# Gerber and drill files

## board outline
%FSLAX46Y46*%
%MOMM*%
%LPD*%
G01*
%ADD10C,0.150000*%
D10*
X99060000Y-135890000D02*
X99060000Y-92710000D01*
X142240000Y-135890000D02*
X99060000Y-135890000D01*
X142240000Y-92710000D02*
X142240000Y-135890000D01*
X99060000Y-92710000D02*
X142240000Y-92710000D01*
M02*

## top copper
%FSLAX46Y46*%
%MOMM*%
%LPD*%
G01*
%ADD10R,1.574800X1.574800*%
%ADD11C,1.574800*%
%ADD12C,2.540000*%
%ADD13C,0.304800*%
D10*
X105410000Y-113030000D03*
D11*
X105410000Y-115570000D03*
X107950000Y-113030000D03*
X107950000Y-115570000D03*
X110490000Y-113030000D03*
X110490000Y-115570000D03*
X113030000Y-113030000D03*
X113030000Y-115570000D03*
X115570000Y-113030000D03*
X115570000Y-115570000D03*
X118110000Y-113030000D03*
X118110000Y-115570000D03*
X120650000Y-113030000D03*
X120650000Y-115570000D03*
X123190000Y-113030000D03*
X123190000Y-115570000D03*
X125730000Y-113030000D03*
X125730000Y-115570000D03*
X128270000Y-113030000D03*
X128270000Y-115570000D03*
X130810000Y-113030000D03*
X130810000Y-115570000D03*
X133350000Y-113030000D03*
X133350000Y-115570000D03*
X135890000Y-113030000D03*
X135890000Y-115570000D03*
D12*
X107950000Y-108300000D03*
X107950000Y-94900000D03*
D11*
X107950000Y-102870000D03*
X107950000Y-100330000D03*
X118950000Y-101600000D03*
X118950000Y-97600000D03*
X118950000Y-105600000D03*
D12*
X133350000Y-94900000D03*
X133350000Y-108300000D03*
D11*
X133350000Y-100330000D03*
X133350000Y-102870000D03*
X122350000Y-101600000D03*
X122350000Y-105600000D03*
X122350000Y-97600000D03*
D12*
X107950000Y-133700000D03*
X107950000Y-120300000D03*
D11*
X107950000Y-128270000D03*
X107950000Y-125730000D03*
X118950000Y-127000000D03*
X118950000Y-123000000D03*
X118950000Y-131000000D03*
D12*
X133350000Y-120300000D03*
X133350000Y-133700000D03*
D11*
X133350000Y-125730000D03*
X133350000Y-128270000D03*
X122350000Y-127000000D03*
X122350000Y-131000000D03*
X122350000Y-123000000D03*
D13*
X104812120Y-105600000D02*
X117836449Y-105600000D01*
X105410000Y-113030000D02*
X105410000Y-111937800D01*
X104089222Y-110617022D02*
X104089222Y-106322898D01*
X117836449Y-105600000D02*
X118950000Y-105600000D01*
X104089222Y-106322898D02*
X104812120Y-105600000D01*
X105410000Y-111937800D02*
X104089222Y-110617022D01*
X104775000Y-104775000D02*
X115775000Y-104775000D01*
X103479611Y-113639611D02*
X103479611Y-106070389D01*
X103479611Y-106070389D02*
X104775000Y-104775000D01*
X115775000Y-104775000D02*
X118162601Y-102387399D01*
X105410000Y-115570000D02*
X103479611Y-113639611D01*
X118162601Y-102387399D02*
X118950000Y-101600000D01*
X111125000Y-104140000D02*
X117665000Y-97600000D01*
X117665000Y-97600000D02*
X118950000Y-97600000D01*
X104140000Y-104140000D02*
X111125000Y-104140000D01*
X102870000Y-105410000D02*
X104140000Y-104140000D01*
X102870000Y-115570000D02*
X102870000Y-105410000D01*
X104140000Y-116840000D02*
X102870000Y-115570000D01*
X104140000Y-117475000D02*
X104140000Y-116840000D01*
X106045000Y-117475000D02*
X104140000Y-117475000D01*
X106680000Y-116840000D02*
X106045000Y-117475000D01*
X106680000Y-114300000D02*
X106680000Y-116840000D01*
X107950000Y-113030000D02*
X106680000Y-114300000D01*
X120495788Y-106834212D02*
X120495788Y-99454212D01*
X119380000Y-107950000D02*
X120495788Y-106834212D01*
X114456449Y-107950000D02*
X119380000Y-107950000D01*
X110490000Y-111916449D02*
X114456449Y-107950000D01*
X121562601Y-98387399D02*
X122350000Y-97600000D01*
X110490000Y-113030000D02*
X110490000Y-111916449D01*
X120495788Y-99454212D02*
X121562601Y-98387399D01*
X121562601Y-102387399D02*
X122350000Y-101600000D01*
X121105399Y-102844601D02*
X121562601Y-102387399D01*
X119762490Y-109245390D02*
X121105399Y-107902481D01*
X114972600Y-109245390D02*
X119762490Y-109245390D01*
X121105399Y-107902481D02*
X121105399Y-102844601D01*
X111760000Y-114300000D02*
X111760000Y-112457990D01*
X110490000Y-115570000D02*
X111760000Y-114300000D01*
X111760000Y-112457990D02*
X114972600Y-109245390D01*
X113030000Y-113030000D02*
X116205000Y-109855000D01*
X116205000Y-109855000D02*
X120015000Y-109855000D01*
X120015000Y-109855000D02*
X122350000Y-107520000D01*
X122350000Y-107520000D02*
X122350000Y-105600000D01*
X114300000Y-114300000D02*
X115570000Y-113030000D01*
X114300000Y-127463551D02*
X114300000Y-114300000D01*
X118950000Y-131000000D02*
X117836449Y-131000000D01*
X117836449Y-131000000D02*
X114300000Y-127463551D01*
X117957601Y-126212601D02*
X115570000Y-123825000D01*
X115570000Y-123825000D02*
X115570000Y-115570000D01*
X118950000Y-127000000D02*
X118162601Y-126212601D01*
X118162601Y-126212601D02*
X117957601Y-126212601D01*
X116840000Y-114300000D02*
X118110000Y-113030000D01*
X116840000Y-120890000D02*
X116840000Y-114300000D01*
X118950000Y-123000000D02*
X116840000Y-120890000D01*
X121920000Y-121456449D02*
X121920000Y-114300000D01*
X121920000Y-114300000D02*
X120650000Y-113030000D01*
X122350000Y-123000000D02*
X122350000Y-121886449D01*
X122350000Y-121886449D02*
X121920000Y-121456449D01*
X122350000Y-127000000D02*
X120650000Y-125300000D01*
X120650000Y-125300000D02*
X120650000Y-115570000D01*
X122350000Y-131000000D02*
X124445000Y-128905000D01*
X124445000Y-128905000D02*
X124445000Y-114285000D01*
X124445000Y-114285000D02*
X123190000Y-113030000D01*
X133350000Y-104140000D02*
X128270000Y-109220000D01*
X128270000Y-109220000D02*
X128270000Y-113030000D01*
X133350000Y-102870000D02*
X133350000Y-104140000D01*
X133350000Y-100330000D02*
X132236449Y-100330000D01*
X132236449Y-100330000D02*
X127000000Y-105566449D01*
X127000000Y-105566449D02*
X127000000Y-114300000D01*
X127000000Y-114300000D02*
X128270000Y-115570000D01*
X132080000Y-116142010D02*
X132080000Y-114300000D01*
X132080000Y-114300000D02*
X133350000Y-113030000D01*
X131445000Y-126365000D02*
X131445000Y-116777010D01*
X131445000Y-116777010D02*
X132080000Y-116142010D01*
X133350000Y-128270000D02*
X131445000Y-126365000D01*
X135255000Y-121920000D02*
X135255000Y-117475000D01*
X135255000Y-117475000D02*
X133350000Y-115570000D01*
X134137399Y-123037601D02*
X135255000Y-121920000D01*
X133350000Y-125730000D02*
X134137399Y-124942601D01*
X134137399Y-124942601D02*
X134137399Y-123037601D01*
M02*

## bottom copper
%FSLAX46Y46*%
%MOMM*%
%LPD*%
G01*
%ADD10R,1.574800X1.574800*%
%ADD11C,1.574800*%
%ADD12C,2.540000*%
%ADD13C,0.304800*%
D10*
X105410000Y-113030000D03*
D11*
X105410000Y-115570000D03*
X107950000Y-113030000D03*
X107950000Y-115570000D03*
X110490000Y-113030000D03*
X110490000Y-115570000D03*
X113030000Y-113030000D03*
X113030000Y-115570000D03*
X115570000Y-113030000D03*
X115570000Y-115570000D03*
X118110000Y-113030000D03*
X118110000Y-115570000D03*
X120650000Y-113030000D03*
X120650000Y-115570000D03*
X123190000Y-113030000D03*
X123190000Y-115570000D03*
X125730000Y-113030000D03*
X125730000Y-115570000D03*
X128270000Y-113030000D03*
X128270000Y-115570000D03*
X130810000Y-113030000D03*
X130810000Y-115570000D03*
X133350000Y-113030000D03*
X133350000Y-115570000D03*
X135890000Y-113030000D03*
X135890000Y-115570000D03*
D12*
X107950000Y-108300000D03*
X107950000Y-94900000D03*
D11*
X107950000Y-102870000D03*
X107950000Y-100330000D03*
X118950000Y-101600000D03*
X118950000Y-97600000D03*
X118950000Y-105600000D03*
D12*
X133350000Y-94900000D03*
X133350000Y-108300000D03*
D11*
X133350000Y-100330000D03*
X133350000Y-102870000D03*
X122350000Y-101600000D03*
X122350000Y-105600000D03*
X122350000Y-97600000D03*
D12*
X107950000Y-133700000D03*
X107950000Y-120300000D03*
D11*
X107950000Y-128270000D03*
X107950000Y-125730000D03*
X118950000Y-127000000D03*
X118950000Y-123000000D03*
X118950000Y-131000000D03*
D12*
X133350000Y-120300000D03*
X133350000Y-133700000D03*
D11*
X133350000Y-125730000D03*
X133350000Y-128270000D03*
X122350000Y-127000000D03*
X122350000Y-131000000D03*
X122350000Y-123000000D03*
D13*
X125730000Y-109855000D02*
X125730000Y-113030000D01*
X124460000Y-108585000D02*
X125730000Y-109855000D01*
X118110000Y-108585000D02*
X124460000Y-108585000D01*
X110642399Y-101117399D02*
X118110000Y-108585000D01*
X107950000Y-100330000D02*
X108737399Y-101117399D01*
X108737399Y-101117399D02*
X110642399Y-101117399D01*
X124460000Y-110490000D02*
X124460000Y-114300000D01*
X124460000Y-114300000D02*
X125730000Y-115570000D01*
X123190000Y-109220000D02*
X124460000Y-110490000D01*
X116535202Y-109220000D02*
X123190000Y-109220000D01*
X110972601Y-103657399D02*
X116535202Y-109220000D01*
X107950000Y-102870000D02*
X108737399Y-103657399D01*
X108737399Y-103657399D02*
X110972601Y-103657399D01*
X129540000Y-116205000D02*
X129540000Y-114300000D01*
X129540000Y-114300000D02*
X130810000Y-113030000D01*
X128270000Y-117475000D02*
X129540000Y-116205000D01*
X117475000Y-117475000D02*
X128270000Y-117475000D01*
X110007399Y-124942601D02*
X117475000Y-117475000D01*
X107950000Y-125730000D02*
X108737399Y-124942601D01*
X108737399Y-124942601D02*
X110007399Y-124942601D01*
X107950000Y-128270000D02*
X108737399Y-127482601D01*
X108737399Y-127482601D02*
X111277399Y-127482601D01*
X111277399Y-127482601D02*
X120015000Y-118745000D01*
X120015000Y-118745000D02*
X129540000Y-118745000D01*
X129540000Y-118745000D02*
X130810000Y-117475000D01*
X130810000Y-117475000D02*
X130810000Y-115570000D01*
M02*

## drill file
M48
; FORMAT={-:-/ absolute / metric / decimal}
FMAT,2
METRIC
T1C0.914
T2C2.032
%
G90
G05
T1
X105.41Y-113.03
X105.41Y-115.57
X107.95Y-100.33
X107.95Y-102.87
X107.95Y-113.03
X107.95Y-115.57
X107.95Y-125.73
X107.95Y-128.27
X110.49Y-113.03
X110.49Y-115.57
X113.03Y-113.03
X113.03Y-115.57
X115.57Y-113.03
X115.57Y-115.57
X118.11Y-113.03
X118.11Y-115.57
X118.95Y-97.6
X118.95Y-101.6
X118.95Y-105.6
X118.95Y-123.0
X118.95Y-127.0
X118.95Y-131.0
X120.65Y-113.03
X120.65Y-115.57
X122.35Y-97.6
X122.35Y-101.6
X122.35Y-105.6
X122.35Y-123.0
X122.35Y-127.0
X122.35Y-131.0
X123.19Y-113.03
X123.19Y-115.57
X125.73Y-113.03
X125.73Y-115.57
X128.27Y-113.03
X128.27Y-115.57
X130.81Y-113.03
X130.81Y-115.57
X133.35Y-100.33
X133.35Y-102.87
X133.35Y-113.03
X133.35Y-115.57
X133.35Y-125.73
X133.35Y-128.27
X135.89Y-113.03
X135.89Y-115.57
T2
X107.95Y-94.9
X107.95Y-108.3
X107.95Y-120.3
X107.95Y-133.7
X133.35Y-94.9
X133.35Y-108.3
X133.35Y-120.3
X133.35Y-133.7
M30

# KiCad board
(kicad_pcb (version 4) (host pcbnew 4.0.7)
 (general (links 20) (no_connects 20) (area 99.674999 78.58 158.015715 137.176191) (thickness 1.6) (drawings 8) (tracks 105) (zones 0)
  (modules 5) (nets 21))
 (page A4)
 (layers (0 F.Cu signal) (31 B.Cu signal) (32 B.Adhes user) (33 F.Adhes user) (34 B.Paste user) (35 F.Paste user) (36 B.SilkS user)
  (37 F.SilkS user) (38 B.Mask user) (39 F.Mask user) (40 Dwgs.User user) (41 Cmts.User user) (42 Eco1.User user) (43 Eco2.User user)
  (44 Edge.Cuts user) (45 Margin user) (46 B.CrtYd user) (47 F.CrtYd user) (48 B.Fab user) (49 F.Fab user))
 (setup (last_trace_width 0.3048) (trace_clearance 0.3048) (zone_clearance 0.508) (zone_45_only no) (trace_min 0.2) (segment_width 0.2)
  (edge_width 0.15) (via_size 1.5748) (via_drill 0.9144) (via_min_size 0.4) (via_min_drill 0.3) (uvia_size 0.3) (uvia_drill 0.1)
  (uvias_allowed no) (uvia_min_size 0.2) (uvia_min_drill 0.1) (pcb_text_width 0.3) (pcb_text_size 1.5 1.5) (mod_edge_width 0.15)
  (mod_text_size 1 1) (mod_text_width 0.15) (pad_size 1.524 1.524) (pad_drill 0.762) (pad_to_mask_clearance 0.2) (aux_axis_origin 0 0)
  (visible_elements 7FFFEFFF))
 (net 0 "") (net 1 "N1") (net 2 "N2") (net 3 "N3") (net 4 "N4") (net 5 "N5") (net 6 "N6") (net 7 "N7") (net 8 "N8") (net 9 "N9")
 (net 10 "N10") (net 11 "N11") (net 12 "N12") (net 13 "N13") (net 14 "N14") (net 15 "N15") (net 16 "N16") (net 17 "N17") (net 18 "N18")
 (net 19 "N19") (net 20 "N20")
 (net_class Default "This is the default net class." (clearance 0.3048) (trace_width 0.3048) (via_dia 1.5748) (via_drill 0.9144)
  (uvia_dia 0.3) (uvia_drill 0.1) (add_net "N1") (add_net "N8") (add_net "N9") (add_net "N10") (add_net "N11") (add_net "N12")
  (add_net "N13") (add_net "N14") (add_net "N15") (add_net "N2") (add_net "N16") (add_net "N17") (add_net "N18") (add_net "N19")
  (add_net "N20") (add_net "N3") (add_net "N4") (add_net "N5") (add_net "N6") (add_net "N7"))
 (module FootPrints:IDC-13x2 (layer B.Cu) (at 113.03 113.03)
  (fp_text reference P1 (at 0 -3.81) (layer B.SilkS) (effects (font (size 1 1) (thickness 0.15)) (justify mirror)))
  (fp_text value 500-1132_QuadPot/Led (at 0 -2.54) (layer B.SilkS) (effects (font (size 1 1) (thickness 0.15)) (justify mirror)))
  (pad 1 thru_hole rect (at -7.62 0) (size 1.5748 1.5748) (drill 0.9144) (layers *.Cu *.Mask) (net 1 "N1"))
  (pad 2 thru_hole circle (at -7.62 2.54) (size 1.5748 1.5748) (drill 0.9144) (layers *.Cu *.Mask) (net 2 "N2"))
  (pad 3 thru_hole circle (at -5.08 0) (size 1.5748 1.5748) (drill 0.9144) (layers *.Cu *.Mask) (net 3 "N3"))
  (pad 4 thru_hole circle (at -5.08 2.54) (size 1.5748 1.5748) (drill 0.9144) (layers *.Cu *.Mask))
  (pad 5 thru_hole circle (at -2.54 0) (size 1.5748 1.5748) (drill 0.9144) (layers *.Cu *.Mask) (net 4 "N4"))
  (pad 6 thru_hole circle (at -2.54 2.54) (size 1.5748 1.5748) (drill 0.9144) (layers *.Cu *.Mask) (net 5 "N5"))
  (pad 7 thru_hole circle (at 0 0) (size 1.5748 1.5748) (drill 0.9144) (layers *.Cu *.Mask) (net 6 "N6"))
  (pad 8 thru_hole circle (at 0 2.54) (size 1.5748 1.5748) (drill 0.9144) (layers *.Cu *.Mask))
  (pad 9 thru_hole circle (at 2.54 0) (size 1.5748 1.5748) (drill 0.9144) (layers *.Cu *.Mask) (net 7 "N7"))
  (pad 10 thru_hole circle (at 2.54 2.54) (size 1.5748 1.5748) (drill 0.9144) (layers *.Cu *.Mask) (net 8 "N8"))
  (pad 11 thru_hole circle (at 5.08 0) (size 1.5748 1.5748) (drill 0.9144) (layers *.Cu *.Mask) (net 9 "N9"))
  (pad 12 thru_hole circle (at 5.08 2.54) (size 1.5748 1.5748) (drill 0.9144) (layers *.Cu *.Mask))
  (pad 13 thru_hole circle (at 7.62 0) (size 1.5748 1.5748) (drill 0.9144) (layers *.Cu *.Mask) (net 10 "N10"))
  (pad 14 thru_hole circle (at 7.62 2.54) (size 1.5748 1.5748) (drill 0.9144) (layers *.Cu *.Mask) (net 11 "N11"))
  (pad 15 thru_hole circle (at 10.16 0) (size 1.5748 1.5748) (drill 0.9144) (layers *.Cu *.Mask) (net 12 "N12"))
  (pad 16 thru_hole circle (at 10.16 2.54) (size 1.5748 1.5748) (drill 0.9144) (layers *.Cu *.Mask))
  (pad 17 thru_hole circle (at 12.7 0) (size 1.5748 1.5748) (drill 0.9144) (layers *.Cu *.Mask) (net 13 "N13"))
  (pad 18 thru_hole circle (at 12.7 2.54) (size 1.5748 1.5748) (drill 0.9144) (layers *.Cu *.Mask) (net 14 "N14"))
  (pad 19 thru_hole circle (at 15.24 0) (size 1.5748 1.5748) (drill 0.9144) (layers *.Cu *.Mask) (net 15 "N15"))
  (pad 20 thru_hole circle (at 15.24 2.54) (size 1.5748 1.5748) (drill 0.9144) (layers *.Cu *.Mask) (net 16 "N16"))
  (pad 21 thru_hole circle (at 17.78 0) (size 1.5748 1.5748) (drill 0.9144) (layers *.Cu *.Mask) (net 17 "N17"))
  (pad 22 thru_hole circle (at 17.78 2.54) (size 1.5748 1.5748) (drill 0.9144) (layers *.Cu *.Mask) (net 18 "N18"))
  (pad 23 thru_hole circle (at 20.32 0) (size 1.5748 1.5748) (drill 0.9144) (layers *.Cu *.Mask) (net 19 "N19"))
  (pad 24 thru_hole circle (at 20.32 2.54) (size 1.5748 1.5748) (drill 0.9144) (layers *.Cu *.Mask) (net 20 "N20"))
  (pad 25 thru_hole circle (at 22.86 0) (size 1.5748 1.5748) (drill 0.9144) (layers *.Cu *.Mask))
  (pad 26 thru_hole circle (at 22.86 2.54) (size 1.5748 1.5748) (drill 0.9144) (layers *.Cu *.Mask)))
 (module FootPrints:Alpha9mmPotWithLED (layer F.Cu) (at 107.95 101.6 90)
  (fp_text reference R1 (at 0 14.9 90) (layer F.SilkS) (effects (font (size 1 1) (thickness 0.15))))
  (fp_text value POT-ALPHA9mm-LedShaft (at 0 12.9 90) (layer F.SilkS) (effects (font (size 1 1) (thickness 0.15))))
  (pad "" thru_hole circle (at -6.7 0 90) (size 2.54 2.54) (drill 2.032) (layers *.Cu *.Mask F.SilkS))
  (pad "" thru_hole circle (at 6.7 0 90) (size 2.54 2.54) (drill 2.032) (layers *.Cu *.Mask F.SilkS))
  (pad 4 thru_hole circle (at -1.27 0 90) (size 1.5748 1.5748) (drill 0.9144) (layers *.Cu *.Mask F.SilkS) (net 14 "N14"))
  (pad 5 thru_hole circle (at 1.27 0 90) (size 1.5748 1.5748) (drill 0.9144) (layers *.Cu *.Mask F.SilkS) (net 13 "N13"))
  (pad 2 thru_hole circle (at 0 11 90) (size 1.5748 1.5748) (drill 0.9144) (layers *.Cu *.Mask F.SilkS) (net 2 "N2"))
  (pad 3 thru_hole circle (at 4 11 90) (size 1.5748 1.5748) (drill 0.9144) (layers *.Cu *.Mask F.SilkS) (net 3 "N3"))
  (pad 1 thru_hole circle (at -4 11 90) (size 1.5748 1.5748) (drill 0.9144) (layers *.Cu *.Mask F.SilkS) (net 1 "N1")))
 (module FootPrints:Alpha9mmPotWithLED (layer F.Cu) (at 133.35 101.6 270)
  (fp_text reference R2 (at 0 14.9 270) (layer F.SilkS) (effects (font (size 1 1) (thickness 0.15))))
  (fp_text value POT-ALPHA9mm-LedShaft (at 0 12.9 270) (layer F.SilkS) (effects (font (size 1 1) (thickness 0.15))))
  (pad "" thru_hole circle (at -6.7 0 270) (size 2.54 2.54) (drill 2.032) (layers *.Cu *.Mask F.SilkS))
  (pad "" thru_hole circle (at 6.7 0 270) (size 2.54 2.54) (drill 2.032) (layers *.Cu *.Mask F.SilkS))
  (pad 4 thru_hole circle (at -1.27 0 270) (size 1.5748 1.5748) (drill 0.9144) (layers *.Cu *.Mask F.SilkS) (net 16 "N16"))
  (pad 5 thru_hole circle (at 1.27 0 270) (size 1.5748 1.5748) (drill 0.9144) (layers *.Cu *.Mask F.SilkS) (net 15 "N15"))
  (pad 2 thru_hole circle (at 0 11 270) (size 1.5748 1.5748) (drill 0.9144) (layers *.Cu *.Mask F.SilkS) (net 5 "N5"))
  (pad 3 thru_hole circle (at 4 11 270) (size 1.5748 1.5748) (drill 0.9144) (layers *.Cu *.Mask F.SilkS) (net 6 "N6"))
  (pad 1 thru_hole circle (at -4 11 270) (size 1.5748 1.5748) (drill 0.9144) (layers *.Cu *.Mask F.SilkS) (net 4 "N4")))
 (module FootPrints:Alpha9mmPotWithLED (layer F.Cu) (at 107.95 127 90)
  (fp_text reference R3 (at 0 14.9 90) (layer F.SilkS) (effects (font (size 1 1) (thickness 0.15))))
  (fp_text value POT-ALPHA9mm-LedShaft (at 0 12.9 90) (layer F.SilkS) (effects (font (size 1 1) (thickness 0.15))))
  (pad "" thru_hole circle (at -6.7 0 90) (size 2.54 2.54) (drill 2.032) (layers *.Cu *.Mask F.SilkS))
  (pad "" thru_hole circle (at 6.7 0 90) (size 2.54 2.54) (drill 2.032) (layers *.Cu *.Mask F.SilkS))
  (pad 4 thru_hole circle (at -1.27 0 90) (size 1.5748 1.5748) (drill 0.9144) (layers *.Cu *.Mask F.SilkS) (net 18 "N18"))
  (pad 5 thru_hole circle (at 1.27 0 90) (size 1.5748 1.5748) (drill 0.9144) (layers *.Cu *.Mask F.SilkS) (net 17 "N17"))
  (pad 2 thru_hole circle (at 0 11 90) (size 1.5748 1.5748) (drill 0.9144) (layers *.Cu *.Mask F.SilkS) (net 8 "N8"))
  (pad 3 thru_hole circle (at 4 11 90) (size 1.5748 1.5748) (drill 0.9144) (layers *.Cu *.Mask F.SilkS) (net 9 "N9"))
  (pad 1 thru_hole circle (at -4 11 90) (size 1.5748 1.5748) (drill 0.9144) (layers *.Cu *.Mask F.SilkS) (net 7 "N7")))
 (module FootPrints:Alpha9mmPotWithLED (layer F.Cu) (at 133.35 127 270)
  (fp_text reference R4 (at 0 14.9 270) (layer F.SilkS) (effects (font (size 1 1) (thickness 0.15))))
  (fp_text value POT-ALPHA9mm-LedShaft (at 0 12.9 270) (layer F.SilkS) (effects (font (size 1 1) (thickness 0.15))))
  (pad "" thru_hole circle (at -6.7 0 270) (size 2.54 2.54) (drill 2.032) (layers *.Cu *.Mask F.SilkS))
  (pad "" thru_hole circle (at 6.7 0 270) (size 2.54 2.54) (drill 2.032) (layers *.Cu *.Mask F.SilkS))
  (pad 4 thru_hole circle (at -1.27 0 270) (size 1.5748 1.5748) (drill 0.9144) (layers *.Cu *.Mask F.SilkS) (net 20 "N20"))
  (pad 5 thru_hole circle (at 1.27 0 270) (size 1.5748 1.5748) (drill 0.9144) (layers *.Cu *.Mask F.SilkS) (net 19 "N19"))
  (pad 2 thru_hole circle (at 0 11 270) (size 1.5748 1.5748) (drill 0.9144) (layers *.Cu *.Mask F.SilkS) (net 11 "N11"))
  (pad 3 thru_hole circle (at 4 11 270) (size 1.5748 1.5748) (drill 0.9144) (layers *.Cu *.Mask F.SilkS) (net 12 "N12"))
  (pad 1 thru_hole circle (at -4 11 270) (size 1.5748 1.5748) (drill 0.9144) (layers *.Cu *.Mask F.SilkS) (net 10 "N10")))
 (gr_line (start 99.06 135.89) (end 99.06 92.71) (layer Edge.Cuts) (width 0.15))
 (gr_line (start 142.24 135.89) (end 99.06 135.89) (layer Edge.Cuts) (width 0.15))
 (gr_line (start 142.24 92.71) (end 142.24 135.89) (layer Edge.Cuts) (width 0.15))
 (gr_line (start 99.06 92.71) (end 142.24 92.71) (layer Edge.Cuts) (width 0.15))
 (segment (start 104.81212 105.6) (end 117.836449 105.6) (width 0.3048) (layer F.Cu) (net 1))
 (segment (start 105.41 113.03) (end 105.41 111.9378) (width 0.3048) (layer F.Cu) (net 1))
 (segment (start 104.089222 110.617022) (end 104.089222 106.322898) (width 0.3048) (layer F.Cu) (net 1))
 (segment (start 117.836449 105.6) (end 118.95 105.6) (width 0.3048) (layer F.Cu) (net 1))
 (segment (start 104.089222 106.322898) (end 104.81212 105.6) (width 0.3048) (layer F.Cu) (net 1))
 (segment (start 105.41 111.9378) (end 104.089222 110.617022) (width 0.3048) (layer F.Cu) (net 1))
 (segment (start 104.775 104.775) (end 115.775 104.775) (width 0.3048) (layer F.Cu) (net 2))
 (segment (start 103.479611 113.639611) (end 103.479611 106.070389) (width 0.3048) (layer F.Cu) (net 2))
 (segment (start 103.479611 106.070389) (end 104.775 104.775) (width 0.3048) (layer F.Cu) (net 2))
 (segment (start 115.775 104.775) (end 118.162601 102.387399) (width 0.3048) (layer F.Cu) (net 2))
 (segment (start 105.41 115.57) (end 103.479611 113.639611) (width 0.3048) (layer F.Cu) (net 2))
 (segment (start 118.162601 102.387399) (end 118.95 101.6) (width 0.3048) (layer F.Cu) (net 2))
 (segment (start 111.125 104.14) (end 117.665 97.6) (width 0.3048) (layer F.Cu) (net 3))
 (segment (start 117.665 97.6) (end 118.95 97.6) (width 0.3048) (layer F.Cu) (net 3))
 (segment (start 104.14 104.14) (end 111.125 104.14) (width 0.3048) (layer F.Cu) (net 3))
 (segment (start 102.87 105.41) (end 104.14 104.14) (width 0.3048) (layer F.Cu) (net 3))
 (segment (start 102.87 115.57) (end 102.87 105.41) (width 0.3048) (layer F.Cu) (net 3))
 (segment (start 104.14 116.84) (end 102.87 115.57) (width 0.3048) (layer F.Cu) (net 3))
 (segment (start 104.14 117.475) (end 104.14 116.84) (width 0.3048) (layer F.Cu) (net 3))
 (segment (start 106.045 117.475) (end 104.14 117.475) (width 0.3048) (layer F.Cu) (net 3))
 (segment (start 106.68 116.84) (end 106.045 117.475) (width 0.3048) (layer F.Cu) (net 3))
 (segment (start 106.68 114.3) (end 106.68 116.84) (width 0.3048) (layer F.Cu) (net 3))
 (segment (start 107.95 113.03) (end 106.68 114.3) (width 0.3048) (layer F.Cu) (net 3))
 (segment (start 120.495788 106.834212) (end 120.495788 99.454212) (width 0.3048) (layer F.Cu) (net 4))
 (segment (start 119.38 107.95) (end 120.495788 106.834212) (width 0.3048) (layer F.Cu) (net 4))
 (segment (start 114.456449 107.95) (end 119.38 107.95) (width 0.3048) (layer F.Cu) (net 4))
 (segment (start 110.49 111.916449) (end 114.456449 107.95) (width 0.3048) (layer F.Cu) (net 4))
 (segment (start 121.562601 98.387399) (end 122.35 97.6) (width 0.3048) (layer F.Cu) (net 4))
 (segment (start 110.49 113.03) (end 110.49 111.916449) (width 0.3048) (layer F.Cu) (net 4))
 (segment (start 120.495788 99.454212) (end 121.562601 98.387399) (width 0.3048) (layer F.Cu) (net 4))
 (segment (start 121.562601 102.387399) (end 122.35 101.6) (width 0.3048) (layer F.Cu) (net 5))
 (segment (start 121.105399 102.844601) (end 121.562601 102.387399) (width 0.3048) (layer F.Cu) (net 5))
 (segment (start 119.76249 109.24539) (end 121.105399 107.902481) (width 0.3048) (layer F.Cu) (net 5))
 (segment (start 114.9726 109.24539) (end 119.76249 109.24539) (width 0.3048) (layer F.Cu) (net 5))
 (segment (start 121.105399 107.902481) (end 121.105399 102.844601) (width 0.3048) (layer F.Cu) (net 5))
 (segment (start 111.76 114.3) (end 111.76 112.45799) (width 0.3048) (layer F.Cu) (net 5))
 (segment (start 110.49 115.57) (end 111.76 114.3) (width 0.3048) (layer F.Cu) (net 5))
 (segment (start 111.76 112.45799) (end 114.9726 109.24539) (width 0.3048) (layer F.Cu) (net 5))
 (segment (start 113.03 113.03) (end 116.205 109.855) (width 0.3048) (layer F.Cu) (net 6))
 (segment (start 116.205 109.855) (end 120.015 109.855) (width 0.3048) (layer F.Cu) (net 6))
 (segment (start 120.015 109.855) (end 122.35 107.52) (width 0.3048) (layer F.Cu) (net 6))
 (segment (start 122.35 107.52) (end 122.35 105.6) (width 0.3048) (layer F.Cu) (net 6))
 (segment (start 114.3 114.3) (end 115.57 113.03) (width 0.3048) (layer F.Cu) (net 7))
 (segment (start 114.3 127.463551) (end 114.3 114.3) (width 0.3048) (layer F.Cu) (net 7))
 (segment (start 118.95 131) (end 117.836449 131) (width 0.3048) (layer F.Cu) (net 7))
 (segment (start 117.836449 131) (end 114.3 127.463551) (width 0.3048) (layer F.Cu) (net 7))
 (segment (start 117.957601 126.212601) (end 115.57 123.825) (width 0.3048) (layer F.Cu) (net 8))
 (segment (start 115.57 123.825) (end 115.57 115.57) (width 0.3048) (layer F.Cu) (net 8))
 (segment (start 118.95 127) (end 118.162601 126.212601) (width 0.3048) (layer F.Cu) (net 8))
 (segment (start 118.162601 126.212601) (end 117.957601 126.212601) (width 0.3048) (layer F.Cu) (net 8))
 (segment (start 116.84 114.3) (end 118.11 113.03) (width 0.3048) (layer F.Cu) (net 9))
 (segment (start 116.84 120.89) (end 116.84 114.3) (width 0.3048) (layer F.Cu) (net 9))
 (segment (start 118.95 123) (end 116.84 120.89) (width 0.3048) (layer F.Cu) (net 9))
 (segment (start 121.92 121.456449) (end 121.92 114.3) (width 0.3048) (layer F.Cu) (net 10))
 (segment (start 121.92 114.3) (end 120.65 113.03) (width 0.3048) (layer F.Cu) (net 10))
 (segment (start 122.35 123) (end 122.35 121.886449) (width 0.3048) (layer F.Cu) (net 10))
 (segment (start 122.35 121.886449) (end 121.92 121.456449) (width 0.3048) (layer F.Cu) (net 10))
 (segment (start 122.35 127) (end 120.65 125.3) (width 0.3048) (layer F.Cu) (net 11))
 (segment (start 120.65 125.3) (end 120.65 115.57) (width 0.3048) (layer F.Cu) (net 11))
 (segment (start 122.35 131) (end 124.445 128.905) (width 0.3048) (layer F.Cu) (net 12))
 (segment (start 124.445 128.905) (end 124.445 114.285) (width 0.3048) (layer F.Cu) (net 12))
 (segment (start 124.445 114.285) (end 123.19 113.03) (width 0.3048) (layer F.Cu) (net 12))
 (segment (start 125.73 109.855) (end 125.73 113.03) (width 0.3048) (layer B.Cu) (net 13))
 (segment (start 124.46 108.585) (end 125.73 109.855) (width 0.3048) (layer B.Cu) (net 13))
 (segment (start 118.11 108.585) (end 124.46 108.585) (width 0.3048) (layer B.Cu) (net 13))
 (segment (start 110.642399 101.117399) (end 118.11 108.585) (width 0.3048) (layer B.Cu) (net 13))
 (segment (start 107.95 100.33) (end 108.737399 101.117399) (width 0.3048) (layer B.Cu) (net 13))
 (segment (start 108.737399 101.117399) (end 110.642399 101.117399) (width 0.3048) (layer B.Cu) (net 13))
 (segment (start 124.46 110.49) (end 124.46 114.3) (width 0.3048) (layer B.Cu) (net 14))
 (segment (start 124.46 114.3) (end 125.73 115.57) (width 0.3048) (layer B.Cu) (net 14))
 (segment (start 123.19 109.22) (end 124.46 110.49) (width 0.3048) (layer B.Cu) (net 14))
 (segment (start 116.535202 109.22) (end 123.19 109.22) (width 0.3048) (layer B.Cu) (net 14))
 (segment (start 110.972601 103.657399) (end 116.535202 109.22) (width 0.3048) (layer B.Cu) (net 14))
 (segment (start 107.95 102.87) (end 108.737399 103.657399) (width 0.3048) (layer B.Cu) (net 14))
 (segment (start 108.737399 103.657399) (end 110.972601 103.657399) (width 0.3048) (layer B.Cu) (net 14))
 (segment (start 133.35 104.14) (end 128.27 109.22) (width 0.3048) (layer F.Cu) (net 15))
 (segment (start 128.27 109.22) (end 128.27 113.03) (width 0.3048) (layer F.Cu) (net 15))
 (segment (start 133.35 102.87) (end 133.35 104.14) (width 0.3048) (layer F.Cu) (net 15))
 (segment (start 133.35 100.33) (end 132.236449 100.33) (width 0.3048) (layer F.Cu) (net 16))
 (segment (start 132.236449 100.33) (end 127 105.566449) (width 0.3048) (layer F.Cu) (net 16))
 (segment (start 127 105.566449) (end 127 114.3) (width 0.3048) (layer F.Cu) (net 16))
 (segment (start 127 114.3) (end 128.27 115.57) (width 0.3048) (layer F.Cu) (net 16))
 (segment (start 129.54 116.205) (end 129.54 114.3) (width 0.3048) (layer B.Cu) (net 17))
 (segment (start 129.54 114.3) (end 130.81 113.03) (width 0.3048) (layer B.Cu) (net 17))
 (segment (start 128.27 117.475) (end 129.54 116.205) (width 0.3048) (layer B.Cu) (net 17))
 (segment (start 117.475 117.475) (end 128.27 117.475) (width 0.3048) (layer B.Cu) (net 17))
 (segment (start 110.007399 124.942601) (end 117.475 117.475) (width 0.3048) (layer B.Cu) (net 17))
 (segment (start 107.95 125.73) (end 108.737399 124.942601) (width 0.3048) (layer B.Cu) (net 17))
 (segment (start 108.737399 124.942601) (end 110.007399 124.942601) (width 0.3048) (layer B.Cu) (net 17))
 (segment (start 107.95 128.27) (end 108.737399 127.482601) (width 0.3048) (layer B.Cu) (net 18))
 (segment (start 108.737399 127.482601) (end 111.277399 127.482601) (width 0.3048) (layer B.Cu) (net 18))
 (segment (start 111.277399 127.482601) (end 120.015 118.745) (width 0.3048) (layer B.Cu) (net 18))
 (segment (start 120.015 118.745) (end 129.54 118.745) (width 0.3048) (layer B.Cu) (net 18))
 (segment (start 129.54 118.745) (end 130.81 117.475) (width 0.3048) (layer B.Cu) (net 18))
 (segment (start 130.81 117.475) (end 130.81 115.57) (width 0.3048) (layer B.Cu) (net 18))
 (segment (start 132.08 116.14201) (end 132.08 114.3) (width 0.3048) (layer F.Cu) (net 19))
 (segment (start 132.08 114.3) (end 133.35 113.03) (width 0.3048) (layer F.Cu) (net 19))
 (segment (start 131.445 126.365) (end 131.445 116.77701) (width 0.3048) (layer F.Cu) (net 19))
 (segment (start 131.445 116.77701) (end 132.08 116.14201) (width 0.3048) (layer F.Cu) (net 19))
 (segment (start 133.35 128.27) (end 131.445 126.365) (width 0.3048) (layer F.Cu) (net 19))
 (segment (start 135.255 121.92) (end 135.255 117.475) (width 0.3048) (layer F.Cu) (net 20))
 (segment (start 135.255 117.475) (end 133.35 115.57) (width 0.3048) (layer F.Cu) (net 20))
 (segment (start 134.137399 123.037601) (end 135.255 121.92) (width 0.3048) (layer F.Cu) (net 20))
 (segment (start 133.35 125.73) (end 134.137399 124.942601) (width 0.3048) (layer F.Cu) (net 20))
 (segment (start 134.137399 124.942601) (end 134.137399 123.037601) (width 0.3048) (layer F.Cu) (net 20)))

